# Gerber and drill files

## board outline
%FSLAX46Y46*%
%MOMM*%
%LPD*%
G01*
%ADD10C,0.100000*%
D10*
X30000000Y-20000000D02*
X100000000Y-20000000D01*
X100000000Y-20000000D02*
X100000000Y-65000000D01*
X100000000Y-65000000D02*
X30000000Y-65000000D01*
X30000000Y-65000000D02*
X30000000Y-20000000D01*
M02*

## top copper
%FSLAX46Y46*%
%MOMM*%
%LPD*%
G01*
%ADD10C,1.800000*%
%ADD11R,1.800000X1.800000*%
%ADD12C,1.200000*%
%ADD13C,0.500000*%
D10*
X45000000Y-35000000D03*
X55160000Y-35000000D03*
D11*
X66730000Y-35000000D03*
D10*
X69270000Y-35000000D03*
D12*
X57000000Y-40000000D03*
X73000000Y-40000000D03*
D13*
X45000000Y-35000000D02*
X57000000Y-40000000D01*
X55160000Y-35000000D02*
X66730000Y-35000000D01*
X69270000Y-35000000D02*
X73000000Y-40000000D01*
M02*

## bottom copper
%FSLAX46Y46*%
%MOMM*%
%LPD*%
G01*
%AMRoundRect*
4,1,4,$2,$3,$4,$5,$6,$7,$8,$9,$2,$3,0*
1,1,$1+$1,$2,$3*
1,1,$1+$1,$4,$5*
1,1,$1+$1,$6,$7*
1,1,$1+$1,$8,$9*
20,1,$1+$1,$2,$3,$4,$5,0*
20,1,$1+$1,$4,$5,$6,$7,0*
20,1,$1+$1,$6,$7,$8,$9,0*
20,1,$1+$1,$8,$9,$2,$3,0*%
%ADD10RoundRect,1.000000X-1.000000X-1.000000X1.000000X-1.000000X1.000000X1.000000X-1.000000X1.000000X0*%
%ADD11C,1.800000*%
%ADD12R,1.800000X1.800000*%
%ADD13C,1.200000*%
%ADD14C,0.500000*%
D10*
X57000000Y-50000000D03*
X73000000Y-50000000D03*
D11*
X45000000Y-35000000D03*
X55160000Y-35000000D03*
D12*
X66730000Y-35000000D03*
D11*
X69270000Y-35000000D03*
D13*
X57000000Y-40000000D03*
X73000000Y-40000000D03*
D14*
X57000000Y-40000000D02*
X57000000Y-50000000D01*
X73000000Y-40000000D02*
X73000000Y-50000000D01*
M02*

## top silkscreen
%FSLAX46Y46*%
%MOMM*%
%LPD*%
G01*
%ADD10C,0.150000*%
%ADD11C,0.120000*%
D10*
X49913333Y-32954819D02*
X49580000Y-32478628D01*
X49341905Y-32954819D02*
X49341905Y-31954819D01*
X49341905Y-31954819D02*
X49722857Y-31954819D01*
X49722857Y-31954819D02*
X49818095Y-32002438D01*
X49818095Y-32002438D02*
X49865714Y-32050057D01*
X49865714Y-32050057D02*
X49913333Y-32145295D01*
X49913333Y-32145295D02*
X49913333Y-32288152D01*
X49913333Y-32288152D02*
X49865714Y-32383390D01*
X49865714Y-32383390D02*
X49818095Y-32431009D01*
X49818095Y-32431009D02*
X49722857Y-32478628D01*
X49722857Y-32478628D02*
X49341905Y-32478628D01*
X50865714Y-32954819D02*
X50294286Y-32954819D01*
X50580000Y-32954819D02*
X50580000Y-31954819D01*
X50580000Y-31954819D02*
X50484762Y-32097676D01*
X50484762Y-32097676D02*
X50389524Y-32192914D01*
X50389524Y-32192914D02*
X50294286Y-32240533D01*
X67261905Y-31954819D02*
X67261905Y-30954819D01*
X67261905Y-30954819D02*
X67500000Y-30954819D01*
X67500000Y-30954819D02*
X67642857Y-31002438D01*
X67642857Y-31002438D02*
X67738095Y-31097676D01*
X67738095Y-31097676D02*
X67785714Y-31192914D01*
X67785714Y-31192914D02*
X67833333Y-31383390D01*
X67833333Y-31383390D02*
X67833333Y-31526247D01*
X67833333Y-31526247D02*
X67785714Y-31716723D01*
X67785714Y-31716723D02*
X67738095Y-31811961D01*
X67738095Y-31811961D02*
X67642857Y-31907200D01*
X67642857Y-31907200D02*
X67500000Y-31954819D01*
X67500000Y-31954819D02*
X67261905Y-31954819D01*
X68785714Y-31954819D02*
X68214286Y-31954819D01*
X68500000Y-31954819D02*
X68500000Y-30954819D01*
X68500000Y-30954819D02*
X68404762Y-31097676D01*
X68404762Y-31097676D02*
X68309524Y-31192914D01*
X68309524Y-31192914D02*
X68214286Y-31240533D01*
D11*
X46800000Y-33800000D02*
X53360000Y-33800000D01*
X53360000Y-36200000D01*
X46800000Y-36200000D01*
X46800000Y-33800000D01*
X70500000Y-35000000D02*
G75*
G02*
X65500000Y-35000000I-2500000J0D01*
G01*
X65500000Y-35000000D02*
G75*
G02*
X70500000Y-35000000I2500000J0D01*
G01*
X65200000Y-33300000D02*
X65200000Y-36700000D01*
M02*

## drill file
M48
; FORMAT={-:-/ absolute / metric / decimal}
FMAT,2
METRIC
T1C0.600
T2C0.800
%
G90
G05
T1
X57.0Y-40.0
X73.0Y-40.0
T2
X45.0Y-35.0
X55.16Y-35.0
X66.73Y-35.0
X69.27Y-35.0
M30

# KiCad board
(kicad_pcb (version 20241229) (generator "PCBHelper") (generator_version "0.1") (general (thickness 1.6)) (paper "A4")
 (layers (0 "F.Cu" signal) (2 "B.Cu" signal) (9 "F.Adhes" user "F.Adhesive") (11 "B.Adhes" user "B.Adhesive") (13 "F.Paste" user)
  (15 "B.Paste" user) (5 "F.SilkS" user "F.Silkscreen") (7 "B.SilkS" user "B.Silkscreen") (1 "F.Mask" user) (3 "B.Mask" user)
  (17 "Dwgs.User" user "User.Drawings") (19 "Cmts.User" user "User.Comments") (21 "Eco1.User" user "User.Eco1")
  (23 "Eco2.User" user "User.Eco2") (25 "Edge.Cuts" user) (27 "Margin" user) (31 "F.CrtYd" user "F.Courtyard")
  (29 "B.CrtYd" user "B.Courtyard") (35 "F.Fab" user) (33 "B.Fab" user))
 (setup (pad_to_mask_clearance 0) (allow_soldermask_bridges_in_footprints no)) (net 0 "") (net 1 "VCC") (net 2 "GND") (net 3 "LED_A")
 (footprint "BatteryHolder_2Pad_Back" (layer "B.Cu") (at 65 50)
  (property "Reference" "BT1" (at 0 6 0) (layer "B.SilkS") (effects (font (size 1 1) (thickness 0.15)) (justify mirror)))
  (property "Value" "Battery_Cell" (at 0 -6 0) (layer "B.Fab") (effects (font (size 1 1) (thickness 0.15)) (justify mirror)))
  (pad "1" smd roundrect (at -8 0) (size 4 4) (layers "B.Cu" "B.Paste" "B.Mask") (roundrect_rratio 0.25) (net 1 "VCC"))
  (pad "2" smd roundrect (at 8 0) (size 4 4) (layers "B.Cu" "B.Paste" "B.Mask") (roundrect_rratio 0.25) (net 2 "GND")))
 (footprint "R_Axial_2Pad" (layer "F.Cu") (at 45 35)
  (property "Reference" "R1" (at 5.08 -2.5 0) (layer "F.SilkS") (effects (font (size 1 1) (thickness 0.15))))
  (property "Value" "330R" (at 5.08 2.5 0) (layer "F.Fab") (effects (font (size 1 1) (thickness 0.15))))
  (fp_rect (start 1.8 -1.2) (end 8.36 1.2) (stroke (width 0.12) (type solid)) (fill no) (layer "F.SilkS"))
  (pad "1" thru_hole circle (at 0 0) (size 1.8 1.8) (drill 0.8) (layers "*.Cu" "*.Mask") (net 1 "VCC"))
  (pad "2" thru_hole circle (at 10.16 0) (size 1.8 1.8) (drill 0.8) (layers "*.Cu" "*.Mask") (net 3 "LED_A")))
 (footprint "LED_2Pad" (layer "F.Cu") (at 68 35)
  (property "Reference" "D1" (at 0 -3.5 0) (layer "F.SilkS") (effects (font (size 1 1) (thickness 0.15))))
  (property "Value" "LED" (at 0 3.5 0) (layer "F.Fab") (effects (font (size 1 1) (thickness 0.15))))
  (fp_circle (center 0 0) (end 2.5 0) (stroke (width 0.12) (type solid)) (fill no) (layer "F.SilkS"))
  (fp_line (start -2.8 -1.7) (end -2.8 1.7) (stroke (width 0.12) (type solid)) (layer "F.SilkS"))
  (pad "1" thru_hole rect (at -1.27 0) (size 1.8 1.8) (drill 0.8) (layers "*.Cu" "*.Mask") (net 3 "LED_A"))
  (pad "2" thru_hole circle (at 1.27 0) (size 1.8 1.8) (drill 0.8) (layers "*.Cu" "*.Mask") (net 2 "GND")))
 (gr_line (start 30 20) (end 100 20) (stroke (width 0.1) (type solid)) (layer "Edge.Cuts"))
 (gr_line (start 100 20) (end 100 65) (stroke (width 0.1) (type solid)) (layer "Edge.Cuts"))
 (gr_line (start 100 65) (end 30 65) (stroke (width 0.1) (type solid)) (layer "Edge.Cuts"))
 (gr_line (start 30 65) (end 30 20) (stroke (width 0.1) (type solid)) (layer "Edge.Cuts"))
 (segment (start 45 35) (end 57 40) (width 0.5) (layer "F.Cu") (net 1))
 (via (at 57 40) (size 1.2) (drill 0.6) (layers "F.Cu" "B.Cu") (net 1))
 (segment (start 57 40) (end 57 50) (width 0.5) (layer "B.Cu") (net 1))
 (segment (start 55.16 35) (end 66.73 35) (width 0.5) (layer "F.Cu") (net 3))
 (segment (start 69.27 35) (end 73 40) (width 0.5) (layer "F.Cu") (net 2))
 (via (at 73 40) (size 1.2) (drill 0.6) (layers "F.Cu" "B.Cu") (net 2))
 (segment (start 73 40) (end 73 50) (width 0.5) (layer "B.Cu") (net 2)))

